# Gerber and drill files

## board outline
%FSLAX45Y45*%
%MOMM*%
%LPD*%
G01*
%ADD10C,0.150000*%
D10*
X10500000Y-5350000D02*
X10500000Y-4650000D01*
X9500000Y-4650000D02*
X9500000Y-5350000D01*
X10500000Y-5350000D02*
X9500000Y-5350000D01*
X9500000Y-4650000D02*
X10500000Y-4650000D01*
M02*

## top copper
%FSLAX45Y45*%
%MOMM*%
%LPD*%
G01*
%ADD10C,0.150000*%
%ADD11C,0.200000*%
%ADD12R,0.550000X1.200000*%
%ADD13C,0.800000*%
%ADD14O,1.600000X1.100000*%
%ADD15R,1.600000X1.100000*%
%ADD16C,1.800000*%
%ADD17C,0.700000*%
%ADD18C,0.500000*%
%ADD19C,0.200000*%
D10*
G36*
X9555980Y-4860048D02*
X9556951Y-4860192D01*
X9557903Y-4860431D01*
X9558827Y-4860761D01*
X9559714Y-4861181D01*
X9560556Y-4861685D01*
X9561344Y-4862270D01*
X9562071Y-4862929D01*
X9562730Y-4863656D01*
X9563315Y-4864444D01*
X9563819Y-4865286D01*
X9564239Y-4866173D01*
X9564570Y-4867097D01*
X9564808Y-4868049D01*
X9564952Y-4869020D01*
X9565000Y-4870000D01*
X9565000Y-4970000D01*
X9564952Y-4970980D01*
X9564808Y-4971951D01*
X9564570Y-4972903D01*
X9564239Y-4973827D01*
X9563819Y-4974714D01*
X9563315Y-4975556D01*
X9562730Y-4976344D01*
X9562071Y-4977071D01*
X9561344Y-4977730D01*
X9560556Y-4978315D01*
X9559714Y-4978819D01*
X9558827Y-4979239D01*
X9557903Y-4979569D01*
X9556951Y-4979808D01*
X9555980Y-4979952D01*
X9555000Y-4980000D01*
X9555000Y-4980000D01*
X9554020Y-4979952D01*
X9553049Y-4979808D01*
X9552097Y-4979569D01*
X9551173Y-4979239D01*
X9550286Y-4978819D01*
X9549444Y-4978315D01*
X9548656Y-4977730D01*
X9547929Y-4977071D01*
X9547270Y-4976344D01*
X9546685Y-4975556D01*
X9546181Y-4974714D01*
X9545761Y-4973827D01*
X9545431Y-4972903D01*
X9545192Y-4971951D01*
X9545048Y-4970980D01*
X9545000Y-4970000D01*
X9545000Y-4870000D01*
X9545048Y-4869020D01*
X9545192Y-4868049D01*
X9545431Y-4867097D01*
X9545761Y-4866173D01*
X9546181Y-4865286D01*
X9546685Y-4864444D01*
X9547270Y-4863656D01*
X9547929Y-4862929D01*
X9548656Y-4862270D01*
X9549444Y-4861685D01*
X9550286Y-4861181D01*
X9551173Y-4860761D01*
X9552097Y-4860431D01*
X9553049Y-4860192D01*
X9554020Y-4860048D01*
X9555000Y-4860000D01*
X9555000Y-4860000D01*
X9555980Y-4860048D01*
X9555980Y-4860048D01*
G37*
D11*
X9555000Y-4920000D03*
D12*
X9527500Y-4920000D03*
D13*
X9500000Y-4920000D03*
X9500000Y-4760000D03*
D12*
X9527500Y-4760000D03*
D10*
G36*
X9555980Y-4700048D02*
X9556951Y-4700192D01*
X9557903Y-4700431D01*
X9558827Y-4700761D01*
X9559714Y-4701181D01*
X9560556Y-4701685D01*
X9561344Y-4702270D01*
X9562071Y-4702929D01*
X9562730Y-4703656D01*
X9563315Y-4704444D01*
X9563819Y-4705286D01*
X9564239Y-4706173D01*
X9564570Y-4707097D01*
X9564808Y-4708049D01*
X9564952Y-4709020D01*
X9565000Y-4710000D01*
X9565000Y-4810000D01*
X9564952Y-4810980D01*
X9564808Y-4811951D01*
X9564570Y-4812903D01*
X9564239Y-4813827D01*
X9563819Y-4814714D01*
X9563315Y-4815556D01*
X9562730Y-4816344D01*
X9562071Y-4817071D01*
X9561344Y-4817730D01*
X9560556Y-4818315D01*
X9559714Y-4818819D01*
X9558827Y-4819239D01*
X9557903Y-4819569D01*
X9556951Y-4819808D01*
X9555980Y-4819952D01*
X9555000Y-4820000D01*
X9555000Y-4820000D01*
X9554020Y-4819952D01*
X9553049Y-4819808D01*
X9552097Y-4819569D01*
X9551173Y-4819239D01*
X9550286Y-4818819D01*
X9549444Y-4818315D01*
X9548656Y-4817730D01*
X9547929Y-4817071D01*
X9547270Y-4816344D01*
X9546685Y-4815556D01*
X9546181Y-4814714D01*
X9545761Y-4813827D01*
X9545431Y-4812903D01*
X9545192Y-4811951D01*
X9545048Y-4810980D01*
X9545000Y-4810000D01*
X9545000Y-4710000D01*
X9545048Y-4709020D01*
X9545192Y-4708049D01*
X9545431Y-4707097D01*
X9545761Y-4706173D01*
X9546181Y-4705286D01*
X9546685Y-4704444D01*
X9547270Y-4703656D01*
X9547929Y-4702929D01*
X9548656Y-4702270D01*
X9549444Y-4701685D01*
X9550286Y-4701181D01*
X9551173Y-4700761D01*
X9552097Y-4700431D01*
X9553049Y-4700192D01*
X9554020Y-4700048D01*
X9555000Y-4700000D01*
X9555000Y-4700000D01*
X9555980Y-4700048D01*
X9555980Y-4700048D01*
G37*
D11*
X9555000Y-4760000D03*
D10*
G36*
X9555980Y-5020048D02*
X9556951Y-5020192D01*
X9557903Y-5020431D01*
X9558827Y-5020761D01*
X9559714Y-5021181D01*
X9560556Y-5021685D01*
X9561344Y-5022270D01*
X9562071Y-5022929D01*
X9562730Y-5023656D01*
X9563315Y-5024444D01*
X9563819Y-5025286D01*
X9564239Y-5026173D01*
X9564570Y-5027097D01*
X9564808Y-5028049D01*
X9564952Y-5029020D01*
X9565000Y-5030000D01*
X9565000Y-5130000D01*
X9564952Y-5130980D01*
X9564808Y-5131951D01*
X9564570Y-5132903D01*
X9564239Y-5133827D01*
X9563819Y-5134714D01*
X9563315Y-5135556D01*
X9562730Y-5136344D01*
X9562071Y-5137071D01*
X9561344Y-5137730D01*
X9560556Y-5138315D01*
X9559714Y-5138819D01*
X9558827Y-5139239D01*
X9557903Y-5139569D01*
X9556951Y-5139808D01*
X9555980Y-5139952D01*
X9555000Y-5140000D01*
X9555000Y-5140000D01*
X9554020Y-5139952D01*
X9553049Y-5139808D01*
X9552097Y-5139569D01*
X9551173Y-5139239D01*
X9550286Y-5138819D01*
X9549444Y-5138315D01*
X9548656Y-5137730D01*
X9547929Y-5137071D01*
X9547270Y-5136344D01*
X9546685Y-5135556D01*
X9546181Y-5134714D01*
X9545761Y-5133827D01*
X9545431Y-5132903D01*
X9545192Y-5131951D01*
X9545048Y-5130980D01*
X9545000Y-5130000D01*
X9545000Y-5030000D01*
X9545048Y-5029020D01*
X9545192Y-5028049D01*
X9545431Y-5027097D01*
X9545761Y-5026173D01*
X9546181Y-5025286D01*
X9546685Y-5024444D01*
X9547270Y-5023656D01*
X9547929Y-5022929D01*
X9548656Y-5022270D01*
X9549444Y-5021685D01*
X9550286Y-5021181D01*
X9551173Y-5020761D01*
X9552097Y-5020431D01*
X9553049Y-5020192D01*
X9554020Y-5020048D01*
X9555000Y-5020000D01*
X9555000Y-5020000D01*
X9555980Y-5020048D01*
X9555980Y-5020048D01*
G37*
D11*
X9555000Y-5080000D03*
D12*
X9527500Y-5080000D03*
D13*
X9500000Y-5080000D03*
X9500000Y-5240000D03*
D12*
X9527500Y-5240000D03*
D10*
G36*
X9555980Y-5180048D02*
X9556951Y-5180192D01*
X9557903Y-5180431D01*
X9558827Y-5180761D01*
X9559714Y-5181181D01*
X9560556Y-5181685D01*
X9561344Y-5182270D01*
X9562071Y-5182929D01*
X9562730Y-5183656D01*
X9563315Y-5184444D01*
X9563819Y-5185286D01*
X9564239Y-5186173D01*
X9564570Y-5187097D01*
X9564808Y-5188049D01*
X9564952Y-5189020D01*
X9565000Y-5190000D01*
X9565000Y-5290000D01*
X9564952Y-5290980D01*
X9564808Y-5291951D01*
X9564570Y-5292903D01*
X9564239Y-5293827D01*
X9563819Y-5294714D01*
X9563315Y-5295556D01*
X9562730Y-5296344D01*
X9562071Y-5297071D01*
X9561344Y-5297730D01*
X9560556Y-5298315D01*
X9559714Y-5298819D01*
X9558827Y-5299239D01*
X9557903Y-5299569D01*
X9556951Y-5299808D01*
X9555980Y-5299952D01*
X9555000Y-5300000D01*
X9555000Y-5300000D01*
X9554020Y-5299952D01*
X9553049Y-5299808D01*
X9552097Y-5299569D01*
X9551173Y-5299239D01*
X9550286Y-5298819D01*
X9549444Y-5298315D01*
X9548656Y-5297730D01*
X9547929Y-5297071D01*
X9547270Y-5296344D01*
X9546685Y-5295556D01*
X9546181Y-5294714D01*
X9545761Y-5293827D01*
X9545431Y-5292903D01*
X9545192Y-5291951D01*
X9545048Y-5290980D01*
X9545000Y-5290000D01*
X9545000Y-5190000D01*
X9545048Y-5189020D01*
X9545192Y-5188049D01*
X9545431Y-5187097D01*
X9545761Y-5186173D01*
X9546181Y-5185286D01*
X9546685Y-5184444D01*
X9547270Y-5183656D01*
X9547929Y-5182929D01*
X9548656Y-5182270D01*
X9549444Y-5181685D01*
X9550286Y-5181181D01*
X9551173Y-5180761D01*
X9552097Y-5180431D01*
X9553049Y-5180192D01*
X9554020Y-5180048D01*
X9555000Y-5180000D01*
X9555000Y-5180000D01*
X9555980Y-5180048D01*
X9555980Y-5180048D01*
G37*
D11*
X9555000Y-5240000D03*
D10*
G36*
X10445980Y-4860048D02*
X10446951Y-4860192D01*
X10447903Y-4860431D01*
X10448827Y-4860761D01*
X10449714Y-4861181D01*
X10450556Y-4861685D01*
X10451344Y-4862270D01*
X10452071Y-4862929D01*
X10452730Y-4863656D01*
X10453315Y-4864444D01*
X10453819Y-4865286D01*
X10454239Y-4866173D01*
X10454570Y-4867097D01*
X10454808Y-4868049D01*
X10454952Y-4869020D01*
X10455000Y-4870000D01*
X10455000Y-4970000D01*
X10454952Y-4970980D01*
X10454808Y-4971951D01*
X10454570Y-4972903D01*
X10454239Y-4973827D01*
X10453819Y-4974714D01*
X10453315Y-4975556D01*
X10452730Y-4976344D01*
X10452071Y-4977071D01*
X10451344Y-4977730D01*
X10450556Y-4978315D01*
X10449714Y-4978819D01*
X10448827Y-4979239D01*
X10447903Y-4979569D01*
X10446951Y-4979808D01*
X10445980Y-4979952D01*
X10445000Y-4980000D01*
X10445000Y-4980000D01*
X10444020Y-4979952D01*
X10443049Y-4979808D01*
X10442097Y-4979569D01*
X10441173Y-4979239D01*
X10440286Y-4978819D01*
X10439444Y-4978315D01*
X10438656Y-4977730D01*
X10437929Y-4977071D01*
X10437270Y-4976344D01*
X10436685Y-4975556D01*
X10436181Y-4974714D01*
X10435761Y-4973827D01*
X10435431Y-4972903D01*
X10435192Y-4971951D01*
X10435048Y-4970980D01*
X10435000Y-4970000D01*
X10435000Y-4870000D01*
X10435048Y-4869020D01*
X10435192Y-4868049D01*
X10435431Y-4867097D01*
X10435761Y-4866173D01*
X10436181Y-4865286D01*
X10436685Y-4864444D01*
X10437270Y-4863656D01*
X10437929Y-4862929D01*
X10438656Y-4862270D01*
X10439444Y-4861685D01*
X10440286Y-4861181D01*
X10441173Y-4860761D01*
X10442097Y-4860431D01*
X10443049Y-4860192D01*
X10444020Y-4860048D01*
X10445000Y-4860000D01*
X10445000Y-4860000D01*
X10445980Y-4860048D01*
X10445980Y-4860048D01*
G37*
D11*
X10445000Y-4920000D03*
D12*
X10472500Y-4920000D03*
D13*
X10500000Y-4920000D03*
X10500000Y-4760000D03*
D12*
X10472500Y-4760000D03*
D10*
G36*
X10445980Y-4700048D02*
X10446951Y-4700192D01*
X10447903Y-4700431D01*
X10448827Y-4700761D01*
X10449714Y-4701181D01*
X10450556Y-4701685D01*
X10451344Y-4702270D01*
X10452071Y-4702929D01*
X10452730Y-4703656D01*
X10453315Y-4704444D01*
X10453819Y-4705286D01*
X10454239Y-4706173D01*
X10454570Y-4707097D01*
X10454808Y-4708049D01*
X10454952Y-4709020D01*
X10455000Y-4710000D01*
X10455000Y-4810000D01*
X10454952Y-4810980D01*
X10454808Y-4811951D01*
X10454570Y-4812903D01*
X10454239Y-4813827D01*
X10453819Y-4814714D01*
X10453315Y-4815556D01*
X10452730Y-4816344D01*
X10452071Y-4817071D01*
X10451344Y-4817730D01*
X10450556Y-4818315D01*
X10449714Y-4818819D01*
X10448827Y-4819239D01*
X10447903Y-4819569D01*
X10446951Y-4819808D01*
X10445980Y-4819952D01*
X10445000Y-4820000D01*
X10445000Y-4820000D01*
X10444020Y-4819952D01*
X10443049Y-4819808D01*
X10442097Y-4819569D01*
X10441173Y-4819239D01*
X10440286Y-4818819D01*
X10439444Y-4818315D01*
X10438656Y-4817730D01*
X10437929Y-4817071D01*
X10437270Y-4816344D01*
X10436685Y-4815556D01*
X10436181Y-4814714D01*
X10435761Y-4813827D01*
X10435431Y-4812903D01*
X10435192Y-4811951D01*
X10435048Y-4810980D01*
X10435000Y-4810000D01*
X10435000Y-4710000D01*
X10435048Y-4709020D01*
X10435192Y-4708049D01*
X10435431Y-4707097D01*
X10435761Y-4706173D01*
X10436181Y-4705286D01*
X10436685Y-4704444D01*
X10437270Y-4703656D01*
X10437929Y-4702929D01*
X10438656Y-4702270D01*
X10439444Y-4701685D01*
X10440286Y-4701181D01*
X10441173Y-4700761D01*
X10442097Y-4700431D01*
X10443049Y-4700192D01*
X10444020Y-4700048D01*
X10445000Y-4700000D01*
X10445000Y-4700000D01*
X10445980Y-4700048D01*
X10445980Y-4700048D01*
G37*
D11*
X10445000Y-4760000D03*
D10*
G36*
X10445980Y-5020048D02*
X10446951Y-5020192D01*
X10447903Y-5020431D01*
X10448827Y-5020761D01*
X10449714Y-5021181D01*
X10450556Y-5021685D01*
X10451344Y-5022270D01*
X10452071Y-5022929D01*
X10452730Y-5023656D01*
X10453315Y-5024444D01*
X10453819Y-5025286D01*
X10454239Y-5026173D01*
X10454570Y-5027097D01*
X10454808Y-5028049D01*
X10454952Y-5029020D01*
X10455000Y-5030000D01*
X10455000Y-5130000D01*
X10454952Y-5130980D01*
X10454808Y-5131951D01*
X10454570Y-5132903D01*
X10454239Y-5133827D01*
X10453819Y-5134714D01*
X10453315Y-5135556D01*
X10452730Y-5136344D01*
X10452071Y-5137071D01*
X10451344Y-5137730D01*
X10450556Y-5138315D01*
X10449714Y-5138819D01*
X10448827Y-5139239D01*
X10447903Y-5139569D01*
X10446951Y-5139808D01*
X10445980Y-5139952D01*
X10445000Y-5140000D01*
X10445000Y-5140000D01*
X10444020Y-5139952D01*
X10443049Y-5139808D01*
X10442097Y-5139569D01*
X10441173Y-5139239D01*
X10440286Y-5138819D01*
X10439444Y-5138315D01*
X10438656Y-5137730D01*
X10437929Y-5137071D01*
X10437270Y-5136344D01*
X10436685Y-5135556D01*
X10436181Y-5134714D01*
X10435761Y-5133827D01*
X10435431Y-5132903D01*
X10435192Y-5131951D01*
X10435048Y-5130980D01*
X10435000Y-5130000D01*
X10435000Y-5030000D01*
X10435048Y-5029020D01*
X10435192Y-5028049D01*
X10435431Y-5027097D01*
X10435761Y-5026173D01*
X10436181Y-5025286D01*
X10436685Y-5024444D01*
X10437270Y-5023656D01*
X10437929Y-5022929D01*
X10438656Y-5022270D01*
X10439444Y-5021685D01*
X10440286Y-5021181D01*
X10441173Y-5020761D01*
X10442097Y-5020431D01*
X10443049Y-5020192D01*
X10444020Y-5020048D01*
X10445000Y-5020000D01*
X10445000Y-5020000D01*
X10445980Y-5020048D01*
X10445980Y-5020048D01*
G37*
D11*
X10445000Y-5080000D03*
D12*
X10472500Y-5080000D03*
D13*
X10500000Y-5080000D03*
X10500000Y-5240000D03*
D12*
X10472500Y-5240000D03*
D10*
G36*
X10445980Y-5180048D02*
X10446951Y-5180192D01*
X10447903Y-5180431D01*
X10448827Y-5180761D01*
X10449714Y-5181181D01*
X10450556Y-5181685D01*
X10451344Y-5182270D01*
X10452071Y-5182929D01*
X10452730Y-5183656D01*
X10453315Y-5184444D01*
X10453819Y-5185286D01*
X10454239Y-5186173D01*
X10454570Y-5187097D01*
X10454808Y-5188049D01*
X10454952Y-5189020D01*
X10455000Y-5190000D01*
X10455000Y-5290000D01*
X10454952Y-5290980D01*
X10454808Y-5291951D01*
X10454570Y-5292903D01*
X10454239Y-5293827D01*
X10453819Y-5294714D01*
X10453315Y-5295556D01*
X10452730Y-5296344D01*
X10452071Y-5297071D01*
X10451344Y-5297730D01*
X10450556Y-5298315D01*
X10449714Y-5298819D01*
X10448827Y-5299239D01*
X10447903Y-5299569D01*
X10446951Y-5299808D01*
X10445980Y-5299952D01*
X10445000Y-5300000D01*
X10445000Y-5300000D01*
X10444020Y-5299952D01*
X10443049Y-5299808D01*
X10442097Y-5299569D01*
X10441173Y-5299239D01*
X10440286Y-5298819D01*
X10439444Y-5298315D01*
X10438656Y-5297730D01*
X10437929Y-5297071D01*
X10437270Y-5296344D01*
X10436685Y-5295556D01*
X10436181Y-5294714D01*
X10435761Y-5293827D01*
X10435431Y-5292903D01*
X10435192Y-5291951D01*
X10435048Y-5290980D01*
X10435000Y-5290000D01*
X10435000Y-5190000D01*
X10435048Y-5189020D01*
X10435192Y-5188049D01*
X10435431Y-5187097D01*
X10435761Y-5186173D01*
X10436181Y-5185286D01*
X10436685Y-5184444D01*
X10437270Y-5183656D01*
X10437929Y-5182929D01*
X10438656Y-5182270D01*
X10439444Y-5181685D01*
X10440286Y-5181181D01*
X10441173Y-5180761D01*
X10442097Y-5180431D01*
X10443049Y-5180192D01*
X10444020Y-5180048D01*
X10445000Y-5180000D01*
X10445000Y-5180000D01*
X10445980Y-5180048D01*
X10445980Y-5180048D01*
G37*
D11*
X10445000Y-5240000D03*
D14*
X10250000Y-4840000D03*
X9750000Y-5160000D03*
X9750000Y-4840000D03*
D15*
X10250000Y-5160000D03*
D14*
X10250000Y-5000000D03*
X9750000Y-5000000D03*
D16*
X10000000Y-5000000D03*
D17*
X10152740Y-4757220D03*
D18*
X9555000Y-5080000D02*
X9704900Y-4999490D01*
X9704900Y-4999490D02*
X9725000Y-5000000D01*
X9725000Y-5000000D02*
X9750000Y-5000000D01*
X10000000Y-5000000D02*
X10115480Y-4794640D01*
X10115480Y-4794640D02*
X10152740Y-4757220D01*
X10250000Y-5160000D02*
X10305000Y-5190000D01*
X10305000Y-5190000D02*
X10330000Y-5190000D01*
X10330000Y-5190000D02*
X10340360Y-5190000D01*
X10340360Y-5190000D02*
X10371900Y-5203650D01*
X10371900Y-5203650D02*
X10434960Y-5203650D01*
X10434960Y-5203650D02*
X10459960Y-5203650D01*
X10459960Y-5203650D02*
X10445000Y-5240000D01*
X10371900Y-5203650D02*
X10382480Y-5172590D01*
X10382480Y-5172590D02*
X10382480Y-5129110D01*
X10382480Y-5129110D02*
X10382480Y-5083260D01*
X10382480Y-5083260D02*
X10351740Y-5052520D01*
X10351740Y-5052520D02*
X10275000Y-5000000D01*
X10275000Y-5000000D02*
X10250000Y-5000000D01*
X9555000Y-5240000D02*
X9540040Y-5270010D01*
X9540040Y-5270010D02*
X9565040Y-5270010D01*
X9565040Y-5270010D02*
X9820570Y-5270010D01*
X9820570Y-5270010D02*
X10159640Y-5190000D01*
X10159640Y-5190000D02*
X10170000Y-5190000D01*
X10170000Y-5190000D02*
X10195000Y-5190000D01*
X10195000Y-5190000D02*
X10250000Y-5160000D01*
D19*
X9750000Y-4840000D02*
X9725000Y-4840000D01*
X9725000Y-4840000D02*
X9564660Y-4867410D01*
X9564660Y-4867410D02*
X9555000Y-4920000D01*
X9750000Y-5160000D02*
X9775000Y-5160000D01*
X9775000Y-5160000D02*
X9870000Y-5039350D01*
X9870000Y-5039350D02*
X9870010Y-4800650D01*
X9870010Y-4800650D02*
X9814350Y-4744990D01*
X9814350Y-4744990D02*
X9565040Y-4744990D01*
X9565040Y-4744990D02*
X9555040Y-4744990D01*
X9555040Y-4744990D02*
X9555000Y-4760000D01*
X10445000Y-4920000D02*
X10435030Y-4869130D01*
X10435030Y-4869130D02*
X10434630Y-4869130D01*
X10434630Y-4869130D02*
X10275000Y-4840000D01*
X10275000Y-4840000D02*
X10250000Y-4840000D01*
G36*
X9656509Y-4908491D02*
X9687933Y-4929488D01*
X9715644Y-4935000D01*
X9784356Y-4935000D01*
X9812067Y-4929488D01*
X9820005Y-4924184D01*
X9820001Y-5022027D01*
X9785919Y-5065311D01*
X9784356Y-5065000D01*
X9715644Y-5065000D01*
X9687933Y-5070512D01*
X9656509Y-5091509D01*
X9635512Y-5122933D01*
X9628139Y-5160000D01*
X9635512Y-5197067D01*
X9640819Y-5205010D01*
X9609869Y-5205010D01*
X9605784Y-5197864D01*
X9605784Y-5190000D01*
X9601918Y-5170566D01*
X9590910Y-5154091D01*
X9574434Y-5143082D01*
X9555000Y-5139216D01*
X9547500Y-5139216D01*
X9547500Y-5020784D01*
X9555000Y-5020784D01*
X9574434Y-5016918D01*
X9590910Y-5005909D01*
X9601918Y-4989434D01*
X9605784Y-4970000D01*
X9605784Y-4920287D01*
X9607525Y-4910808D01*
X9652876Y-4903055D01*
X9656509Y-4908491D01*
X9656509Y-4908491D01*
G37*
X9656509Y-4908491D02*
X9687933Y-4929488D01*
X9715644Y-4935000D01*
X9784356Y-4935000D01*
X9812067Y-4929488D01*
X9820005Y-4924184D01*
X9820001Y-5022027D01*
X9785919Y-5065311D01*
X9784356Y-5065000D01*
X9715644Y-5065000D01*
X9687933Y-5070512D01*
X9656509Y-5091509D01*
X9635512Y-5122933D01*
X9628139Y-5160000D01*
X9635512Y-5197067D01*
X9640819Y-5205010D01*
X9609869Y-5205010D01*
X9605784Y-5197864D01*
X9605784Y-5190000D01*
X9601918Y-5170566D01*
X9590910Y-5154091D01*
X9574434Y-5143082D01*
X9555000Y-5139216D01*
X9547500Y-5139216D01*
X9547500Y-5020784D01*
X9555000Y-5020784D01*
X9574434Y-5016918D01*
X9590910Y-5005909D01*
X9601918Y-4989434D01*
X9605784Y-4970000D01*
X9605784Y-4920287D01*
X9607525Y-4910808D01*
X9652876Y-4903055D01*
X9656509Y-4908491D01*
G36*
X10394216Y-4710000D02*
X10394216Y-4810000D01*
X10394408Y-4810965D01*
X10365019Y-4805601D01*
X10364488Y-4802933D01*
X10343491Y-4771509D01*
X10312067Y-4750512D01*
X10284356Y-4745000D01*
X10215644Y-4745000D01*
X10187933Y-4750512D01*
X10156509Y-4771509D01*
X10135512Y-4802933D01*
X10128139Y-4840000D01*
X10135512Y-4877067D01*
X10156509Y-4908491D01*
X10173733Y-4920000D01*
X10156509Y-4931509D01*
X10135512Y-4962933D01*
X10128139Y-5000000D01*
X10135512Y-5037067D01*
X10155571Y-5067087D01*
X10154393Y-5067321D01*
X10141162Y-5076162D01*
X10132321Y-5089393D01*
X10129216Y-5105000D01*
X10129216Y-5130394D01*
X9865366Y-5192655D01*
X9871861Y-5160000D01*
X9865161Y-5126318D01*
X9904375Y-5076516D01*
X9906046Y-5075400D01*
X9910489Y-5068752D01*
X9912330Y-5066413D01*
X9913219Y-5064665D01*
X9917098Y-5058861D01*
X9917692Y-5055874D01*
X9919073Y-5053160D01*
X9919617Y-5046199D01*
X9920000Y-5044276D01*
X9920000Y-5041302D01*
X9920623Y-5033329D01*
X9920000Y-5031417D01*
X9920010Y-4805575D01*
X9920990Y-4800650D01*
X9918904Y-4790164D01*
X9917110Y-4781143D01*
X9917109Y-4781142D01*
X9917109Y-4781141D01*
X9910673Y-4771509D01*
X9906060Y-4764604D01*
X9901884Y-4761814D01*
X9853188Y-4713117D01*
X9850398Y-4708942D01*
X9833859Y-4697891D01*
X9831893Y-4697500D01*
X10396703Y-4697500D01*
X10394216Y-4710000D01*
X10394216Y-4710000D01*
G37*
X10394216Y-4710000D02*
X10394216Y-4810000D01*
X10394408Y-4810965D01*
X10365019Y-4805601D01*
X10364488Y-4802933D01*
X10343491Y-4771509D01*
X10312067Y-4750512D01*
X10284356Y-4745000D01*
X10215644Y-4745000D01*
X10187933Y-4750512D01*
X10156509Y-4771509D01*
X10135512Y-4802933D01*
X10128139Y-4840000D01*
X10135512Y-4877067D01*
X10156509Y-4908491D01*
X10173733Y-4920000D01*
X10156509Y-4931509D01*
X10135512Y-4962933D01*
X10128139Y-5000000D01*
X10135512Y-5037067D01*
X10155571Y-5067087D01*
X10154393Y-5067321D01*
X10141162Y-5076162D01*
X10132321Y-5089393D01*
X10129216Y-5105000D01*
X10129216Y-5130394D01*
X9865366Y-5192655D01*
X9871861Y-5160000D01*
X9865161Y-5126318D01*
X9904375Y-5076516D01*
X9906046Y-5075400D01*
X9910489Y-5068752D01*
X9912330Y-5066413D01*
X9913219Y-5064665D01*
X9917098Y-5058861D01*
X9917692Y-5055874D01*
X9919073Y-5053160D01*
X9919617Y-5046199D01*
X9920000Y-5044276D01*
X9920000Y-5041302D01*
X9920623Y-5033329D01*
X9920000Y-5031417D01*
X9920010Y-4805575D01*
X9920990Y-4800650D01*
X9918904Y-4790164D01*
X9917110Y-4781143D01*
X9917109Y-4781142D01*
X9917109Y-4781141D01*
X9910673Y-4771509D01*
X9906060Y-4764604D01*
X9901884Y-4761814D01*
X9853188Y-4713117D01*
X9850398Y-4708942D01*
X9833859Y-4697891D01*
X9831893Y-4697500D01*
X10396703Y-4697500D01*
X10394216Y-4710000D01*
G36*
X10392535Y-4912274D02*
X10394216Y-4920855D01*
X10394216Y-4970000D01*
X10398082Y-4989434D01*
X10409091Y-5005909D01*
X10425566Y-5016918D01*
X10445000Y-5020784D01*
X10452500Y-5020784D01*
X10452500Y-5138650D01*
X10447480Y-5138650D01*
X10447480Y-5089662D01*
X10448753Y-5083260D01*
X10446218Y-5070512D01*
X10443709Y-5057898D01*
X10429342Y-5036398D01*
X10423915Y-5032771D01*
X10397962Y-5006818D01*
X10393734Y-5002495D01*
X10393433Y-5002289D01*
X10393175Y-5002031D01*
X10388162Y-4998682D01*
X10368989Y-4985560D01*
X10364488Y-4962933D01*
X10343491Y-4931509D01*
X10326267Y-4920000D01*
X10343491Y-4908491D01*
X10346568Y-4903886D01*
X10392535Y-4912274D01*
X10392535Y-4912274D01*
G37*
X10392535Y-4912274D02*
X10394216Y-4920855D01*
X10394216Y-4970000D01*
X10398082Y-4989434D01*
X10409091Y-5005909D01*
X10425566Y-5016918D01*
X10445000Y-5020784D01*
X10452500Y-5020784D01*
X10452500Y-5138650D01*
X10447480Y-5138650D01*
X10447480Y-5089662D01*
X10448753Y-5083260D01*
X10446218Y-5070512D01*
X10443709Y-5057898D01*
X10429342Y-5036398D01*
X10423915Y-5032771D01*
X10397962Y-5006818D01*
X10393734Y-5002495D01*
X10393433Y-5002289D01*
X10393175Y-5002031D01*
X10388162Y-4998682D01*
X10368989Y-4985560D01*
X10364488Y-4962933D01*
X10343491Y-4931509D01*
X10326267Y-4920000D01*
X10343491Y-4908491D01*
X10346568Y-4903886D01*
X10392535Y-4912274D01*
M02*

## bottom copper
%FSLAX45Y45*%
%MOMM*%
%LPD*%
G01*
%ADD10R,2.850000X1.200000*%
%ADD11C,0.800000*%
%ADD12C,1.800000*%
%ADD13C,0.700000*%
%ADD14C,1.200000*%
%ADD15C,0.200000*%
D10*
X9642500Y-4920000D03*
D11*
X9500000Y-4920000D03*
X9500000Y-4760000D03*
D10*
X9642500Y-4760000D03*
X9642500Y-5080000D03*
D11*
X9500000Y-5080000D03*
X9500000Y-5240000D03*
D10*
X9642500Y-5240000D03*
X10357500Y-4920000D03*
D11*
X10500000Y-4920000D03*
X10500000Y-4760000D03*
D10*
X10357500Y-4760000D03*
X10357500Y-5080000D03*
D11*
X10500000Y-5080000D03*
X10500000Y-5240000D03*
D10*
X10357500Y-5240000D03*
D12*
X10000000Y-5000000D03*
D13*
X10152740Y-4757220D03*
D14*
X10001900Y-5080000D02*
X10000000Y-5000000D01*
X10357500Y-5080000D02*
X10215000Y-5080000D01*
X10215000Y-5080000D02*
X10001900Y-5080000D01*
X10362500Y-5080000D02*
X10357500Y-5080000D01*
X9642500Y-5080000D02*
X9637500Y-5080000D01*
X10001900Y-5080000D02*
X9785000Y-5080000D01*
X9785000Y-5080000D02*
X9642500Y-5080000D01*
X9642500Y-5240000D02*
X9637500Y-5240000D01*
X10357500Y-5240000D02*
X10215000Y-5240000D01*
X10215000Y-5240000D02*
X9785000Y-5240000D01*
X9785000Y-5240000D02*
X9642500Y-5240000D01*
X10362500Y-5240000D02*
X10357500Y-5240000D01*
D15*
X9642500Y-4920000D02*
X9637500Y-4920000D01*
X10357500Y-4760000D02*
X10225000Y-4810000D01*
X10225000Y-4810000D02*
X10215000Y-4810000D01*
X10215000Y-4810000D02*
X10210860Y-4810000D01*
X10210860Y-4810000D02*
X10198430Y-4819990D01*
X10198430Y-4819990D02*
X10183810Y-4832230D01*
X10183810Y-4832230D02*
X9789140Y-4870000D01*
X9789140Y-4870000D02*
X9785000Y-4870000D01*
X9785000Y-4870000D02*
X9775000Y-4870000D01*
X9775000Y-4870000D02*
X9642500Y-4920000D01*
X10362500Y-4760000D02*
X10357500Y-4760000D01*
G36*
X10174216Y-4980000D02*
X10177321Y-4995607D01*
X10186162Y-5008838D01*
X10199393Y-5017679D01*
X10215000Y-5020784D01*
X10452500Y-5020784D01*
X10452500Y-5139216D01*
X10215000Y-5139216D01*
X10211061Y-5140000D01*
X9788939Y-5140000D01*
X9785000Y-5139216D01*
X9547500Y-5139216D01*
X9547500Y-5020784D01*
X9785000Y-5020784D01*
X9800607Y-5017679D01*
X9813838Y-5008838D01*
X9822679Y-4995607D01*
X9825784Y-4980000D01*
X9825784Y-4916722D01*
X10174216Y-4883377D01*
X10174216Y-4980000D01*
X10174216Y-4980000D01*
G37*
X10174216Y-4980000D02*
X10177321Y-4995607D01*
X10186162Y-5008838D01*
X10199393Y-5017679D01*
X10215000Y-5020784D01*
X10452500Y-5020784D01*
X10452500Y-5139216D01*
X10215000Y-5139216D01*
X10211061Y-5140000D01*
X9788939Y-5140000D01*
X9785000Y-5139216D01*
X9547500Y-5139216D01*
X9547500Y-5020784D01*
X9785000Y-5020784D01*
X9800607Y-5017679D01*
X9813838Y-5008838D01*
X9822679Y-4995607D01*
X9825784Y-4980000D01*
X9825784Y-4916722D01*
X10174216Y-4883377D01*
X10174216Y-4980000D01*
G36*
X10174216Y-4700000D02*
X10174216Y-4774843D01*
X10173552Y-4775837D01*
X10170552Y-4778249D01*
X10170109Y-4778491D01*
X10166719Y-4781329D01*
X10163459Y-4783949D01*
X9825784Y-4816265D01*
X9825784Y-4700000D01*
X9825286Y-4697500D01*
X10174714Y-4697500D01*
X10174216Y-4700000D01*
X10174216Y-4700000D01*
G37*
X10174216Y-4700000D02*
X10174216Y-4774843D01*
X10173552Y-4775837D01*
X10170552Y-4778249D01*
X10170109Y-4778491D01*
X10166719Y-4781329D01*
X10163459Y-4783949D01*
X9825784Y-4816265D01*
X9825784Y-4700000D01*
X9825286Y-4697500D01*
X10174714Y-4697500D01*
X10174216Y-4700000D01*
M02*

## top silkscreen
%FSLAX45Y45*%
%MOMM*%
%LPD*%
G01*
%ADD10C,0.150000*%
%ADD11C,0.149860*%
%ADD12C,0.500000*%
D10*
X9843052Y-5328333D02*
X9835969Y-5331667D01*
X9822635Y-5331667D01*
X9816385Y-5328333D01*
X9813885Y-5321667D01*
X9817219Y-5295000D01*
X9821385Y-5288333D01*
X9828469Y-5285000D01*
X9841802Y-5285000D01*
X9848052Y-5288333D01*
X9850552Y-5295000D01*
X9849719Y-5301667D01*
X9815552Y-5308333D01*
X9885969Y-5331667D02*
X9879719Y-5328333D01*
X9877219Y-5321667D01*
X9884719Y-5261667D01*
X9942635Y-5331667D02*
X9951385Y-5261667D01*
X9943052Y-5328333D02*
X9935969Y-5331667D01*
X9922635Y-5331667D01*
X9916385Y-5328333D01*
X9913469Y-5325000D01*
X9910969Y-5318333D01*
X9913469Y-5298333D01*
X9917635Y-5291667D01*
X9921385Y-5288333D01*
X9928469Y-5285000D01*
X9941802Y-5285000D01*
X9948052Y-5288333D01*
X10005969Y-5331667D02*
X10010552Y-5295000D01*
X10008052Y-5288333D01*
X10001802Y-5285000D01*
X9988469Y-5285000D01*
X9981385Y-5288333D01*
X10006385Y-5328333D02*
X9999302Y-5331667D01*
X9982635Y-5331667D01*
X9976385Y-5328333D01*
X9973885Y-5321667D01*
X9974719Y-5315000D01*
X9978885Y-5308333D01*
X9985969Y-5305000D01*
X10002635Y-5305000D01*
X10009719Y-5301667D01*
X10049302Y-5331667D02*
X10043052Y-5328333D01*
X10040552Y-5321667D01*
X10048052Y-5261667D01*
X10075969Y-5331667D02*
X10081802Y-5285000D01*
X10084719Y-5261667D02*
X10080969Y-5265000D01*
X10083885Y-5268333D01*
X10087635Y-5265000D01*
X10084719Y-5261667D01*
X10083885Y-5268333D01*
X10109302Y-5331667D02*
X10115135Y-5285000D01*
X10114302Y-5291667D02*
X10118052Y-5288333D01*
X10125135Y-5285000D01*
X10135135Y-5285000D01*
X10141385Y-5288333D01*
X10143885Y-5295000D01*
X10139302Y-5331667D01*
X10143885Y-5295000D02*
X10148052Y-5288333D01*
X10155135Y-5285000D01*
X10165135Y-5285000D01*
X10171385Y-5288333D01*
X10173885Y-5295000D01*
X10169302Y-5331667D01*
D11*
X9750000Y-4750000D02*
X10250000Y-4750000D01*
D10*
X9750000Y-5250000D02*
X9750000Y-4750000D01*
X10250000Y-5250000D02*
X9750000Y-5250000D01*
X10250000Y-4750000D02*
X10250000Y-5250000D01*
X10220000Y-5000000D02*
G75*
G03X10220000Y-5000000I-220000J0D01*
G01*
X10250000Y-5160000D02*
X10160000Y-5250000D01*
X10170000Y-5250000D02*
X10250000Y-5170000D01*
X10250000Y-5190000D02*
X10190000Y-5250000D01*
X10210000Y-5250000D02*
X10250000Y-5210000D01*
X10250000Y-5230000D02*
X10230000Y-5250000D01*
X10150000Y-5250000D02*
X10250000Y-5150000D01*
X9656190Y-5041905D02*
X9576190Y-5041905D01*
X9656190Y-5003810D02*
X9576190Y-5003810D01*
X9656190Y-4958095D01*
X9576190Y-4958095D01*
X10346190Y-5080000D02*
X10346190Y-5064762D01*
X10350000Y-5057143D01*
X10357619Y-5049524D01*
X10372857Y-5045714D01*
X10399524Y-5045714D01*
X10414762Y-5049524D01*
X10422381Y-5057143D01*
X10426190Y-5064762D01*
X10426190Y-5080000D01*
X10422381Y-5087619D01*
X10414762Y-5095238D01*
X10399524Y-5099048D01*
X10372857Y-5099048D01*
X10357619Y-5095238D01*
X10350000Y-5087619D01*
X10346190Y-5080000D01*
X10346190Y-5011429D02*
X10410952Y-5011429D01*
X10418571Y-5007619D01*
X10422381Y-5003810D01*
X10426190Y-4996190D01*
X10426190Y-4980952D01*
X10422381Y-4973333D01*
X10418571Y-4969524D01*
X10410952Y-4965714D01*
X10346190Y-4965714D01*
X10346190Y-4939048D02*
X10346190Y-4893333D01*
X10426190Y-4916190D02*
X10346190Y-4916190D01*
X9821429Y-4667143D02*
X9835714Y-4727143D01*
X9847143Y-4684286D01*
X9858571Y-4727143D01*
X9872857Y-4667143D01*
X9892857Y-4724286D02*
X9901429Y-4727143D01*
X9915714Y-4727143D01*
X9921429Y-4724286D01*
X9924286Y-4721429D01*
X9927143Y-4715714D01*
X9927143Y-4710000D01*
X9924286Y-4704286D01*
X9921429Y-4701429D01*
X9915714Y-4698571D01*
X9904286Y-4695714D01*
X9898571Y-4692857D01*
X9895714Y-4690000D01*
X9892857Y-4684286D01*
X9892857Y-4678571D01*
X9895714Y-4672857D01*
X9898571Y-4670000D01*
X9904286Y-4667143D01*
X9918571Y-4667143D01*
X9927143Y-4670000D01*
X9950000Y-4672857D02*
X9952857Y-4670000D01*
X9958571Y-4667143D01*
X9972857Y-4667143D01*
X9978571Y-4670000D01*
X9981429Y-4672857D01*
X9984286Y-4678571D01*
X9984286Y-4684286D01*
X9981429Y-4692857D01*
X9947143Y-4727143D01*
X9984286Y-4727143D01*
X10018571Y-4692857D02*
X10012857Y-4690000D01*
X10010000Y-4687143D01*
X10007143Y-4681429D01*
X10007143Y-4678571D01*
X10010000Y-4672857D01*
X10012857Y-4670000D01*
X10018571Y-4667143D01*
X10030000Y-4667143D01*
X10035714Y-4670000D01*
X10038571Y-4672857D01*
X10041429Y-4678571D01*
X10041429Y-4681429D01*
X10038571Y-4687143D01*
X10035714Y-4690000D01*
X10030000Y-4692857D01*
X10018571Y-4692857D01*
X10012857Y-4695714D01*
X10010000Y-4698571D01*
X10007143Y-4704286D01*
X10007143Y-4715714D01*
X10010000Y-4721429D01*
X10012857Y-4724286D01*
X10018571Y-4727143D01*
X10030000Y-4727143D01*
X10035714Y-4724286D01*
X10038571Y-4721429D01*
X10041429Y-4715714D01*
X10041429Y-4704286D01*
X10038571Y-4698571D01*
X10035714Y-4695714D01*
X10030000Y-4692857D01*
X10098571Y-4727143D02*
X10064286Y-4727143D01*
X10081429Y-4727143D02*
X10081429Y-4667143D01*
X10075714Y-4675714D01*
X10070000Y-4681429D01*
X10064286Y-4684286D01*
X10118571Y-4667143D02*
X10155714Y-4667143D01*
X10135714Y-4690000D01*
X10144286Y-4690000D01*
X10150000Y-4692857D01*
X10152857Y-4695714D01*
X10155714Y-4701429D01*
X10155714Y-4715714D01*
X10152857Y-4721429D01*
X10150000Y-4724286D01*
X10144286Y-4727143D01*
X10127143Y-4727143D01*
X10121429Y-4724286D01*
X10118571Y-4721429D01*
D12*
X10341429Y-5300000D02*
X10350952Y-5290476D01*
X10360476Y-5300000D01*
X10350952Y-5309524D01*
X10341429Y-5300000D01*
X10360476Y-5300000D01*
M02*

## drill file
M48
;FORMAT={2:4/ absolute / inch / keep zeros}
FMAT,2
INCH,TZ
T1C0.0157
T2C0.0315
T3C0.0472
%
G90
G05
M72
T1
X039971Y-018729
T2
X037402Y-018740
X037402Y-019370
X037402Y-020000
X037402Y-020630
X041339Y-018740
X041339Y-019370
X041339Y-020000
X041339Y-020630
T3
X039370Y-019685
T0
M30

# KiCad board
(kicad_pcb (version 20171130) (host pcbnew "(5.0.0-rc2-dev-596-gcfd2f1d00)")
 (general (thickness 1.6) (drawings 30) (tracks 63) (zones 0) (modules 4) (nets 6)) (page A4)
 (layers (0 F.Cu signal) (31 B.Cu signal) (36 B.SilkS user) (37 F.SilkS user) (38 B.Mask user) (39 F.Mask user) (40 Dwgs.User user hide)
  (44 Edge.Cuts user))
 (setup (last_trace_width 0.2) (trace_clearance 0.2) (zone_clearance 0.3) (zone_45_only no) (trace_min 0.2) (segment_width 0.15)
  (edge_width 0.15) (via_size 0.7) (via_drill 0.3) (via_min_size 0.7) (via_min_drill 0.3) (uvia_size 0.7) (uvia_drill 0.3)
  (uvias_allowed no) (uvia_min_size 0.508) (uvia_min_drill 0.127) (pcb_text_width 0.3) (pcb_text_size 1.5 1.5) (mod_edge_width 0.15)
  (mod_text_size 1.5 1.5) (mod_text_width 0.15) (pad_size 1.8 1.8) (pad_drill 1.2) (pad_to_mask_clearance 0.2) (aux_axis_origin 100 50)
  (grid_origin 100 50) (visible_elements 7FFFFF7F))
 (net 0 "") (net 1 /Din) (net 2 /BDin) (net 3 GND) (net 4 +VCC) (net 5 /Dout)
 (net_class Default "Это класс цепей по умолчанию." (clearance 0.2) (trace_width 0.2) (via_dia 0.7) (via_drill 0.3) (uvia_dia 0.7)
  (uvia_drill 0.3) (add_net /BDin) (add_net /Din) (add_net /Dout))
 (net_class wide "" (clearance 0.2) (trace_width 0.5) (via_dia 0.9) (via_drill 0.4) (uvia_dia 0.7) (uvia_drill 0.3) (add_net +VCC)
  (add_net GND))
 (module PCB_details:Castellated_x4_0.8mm (layer F.Cu) (at 95 52.4 90)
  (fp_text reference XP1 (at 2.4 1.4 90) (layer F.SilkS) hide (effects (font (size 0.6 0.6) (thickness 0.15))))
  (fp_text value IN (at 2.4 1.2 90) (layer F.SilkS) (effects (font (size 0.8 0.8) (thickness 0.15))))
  (pad 3 smd roundrect (at 3.2 0.55 90) (size 1.2 0.2) (layers F.Cu F.Mask) (roundrect_rratio 0.5) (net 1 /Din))
  (pad 3 smd rect (at 3.2 1.425 90) (size 1.2 2.85) (layers B.Cu B.Mask) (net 1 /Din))
  (pad 3 smd rect (at 3.2 0.275 90) (size 1.2 0.55) (layers F.Cu F.Mask) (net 1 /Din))
  (pad 3 thru_hole circle (at 3.2 0 90) (size 0.8 0.8) (drill 0.8) (layers *.Cu) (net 1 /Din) (clearance 0.001))
  (pad 4 thru_hole circle (at 4.8 0 90) (size 0.8 0.8) (drill 0.8) (layers *.Cu) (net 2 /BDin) (clearance 0.001))
  (pad 4 smd rect (at 4.8 0.275 90) (size 1.2 0.55) (layers F.Cu F.Mask) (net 2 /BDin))
  (pad 4 smd rect (at 4.8 1.425 90) (size 1.2 2.85) (layers B.Cu B.Mask) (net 2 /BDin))
  (pad 4 smd roundrect (at 4.8 0.55 90) (size 1.2 0.2) (layers F.Cu F.Mask) (roundrect_rratio 0.5) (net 2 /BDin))
  (pad 2 smd roundrect (at 1.6 0.55 90) (size 1.2 0.2) (layers F.Cu F.Mask) (roundrect_rratio 0.5) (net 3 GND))
  (pad 2 smd rect (at 1.6 1.425 90) (size 1.2 2.85) (layers B.Cu B.Mask) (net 3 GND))
  (pad 2 smd rect (at 1.6 0.275 90) (size 1.2 0.55) (layers F.Cu F.Mask) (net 3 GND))
  (pad 2 thru_hole circle (at 1.6 0 90) (size 0.8 0.8) (drill 0.8) (layers *.Cu) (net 3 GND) (clearance 0.001))
  (pad 1 thru_hole circle (at 0 0 90) (size 0.8 0.8) (drill 0.8) (layers *.Cu) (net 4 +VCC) (clearance 0.001))
  (pad 1 smd rect (at 0 0.275 90) (size 1.2 0.55) (layers F.Cu F.Mask) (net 4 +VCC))
  (pad 1 smd rect (at 0 1.425 90) (size 1.2 2.85) (layers B.Cu B.Mask) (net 4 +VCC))
  (pad 1 smd roundrect (at 0 0.55 90) (size 1.2 0.2) (layers F.Cu F.Mask) (roundrect_rratio 0.5) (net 4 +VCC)))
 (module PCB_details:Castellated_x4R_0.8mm (layer F.Cu) (at 105 52.4 270)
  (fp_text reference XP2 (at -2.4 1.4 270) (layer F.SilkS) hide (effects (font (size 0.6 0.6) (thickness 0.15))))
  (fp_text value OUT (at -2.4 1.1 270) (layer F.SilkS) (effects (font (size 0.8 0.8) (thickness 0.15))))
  (pad 3 smd roundrect (at -3.2 0.55 270) (size 1.2 0.2) (layers F.Cu F.Mask) (roundrect_rratio 0.5) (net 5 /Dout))
  (pad 3 smd rect (at -3.2 1.425 270) (size 1.2 2.85) (layers B.Cu B.Mask) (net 5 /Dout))
  (pad 3 smd rect (at -3.2 0.275 270) (size 1.2 0.55) (layers F.Cu F.Mask) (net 5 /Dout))
  (pad 3 thru_hole circle (at -3.2 0 270) (size 0.8 0.8) (drill 0.8) (layers *.Cu) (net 5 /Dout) (clearance 0.001))
  (pad 4 thru_hole circle (at -4.8 0 270) (size 0.8 0.8) (drill 0.8) (layers *.Cu) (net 1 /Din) (clearance 0.001))
  (pad 4 smd rect (at -4.8 0.275 270) (size 1.2 0.55) (layers F.Cu F.Mask) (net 1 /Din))
  (pad 4 smd rect (at -4.8 1.425 270) (size 1.2 2.85) (layers B.Cu B.Mask) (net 1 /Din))
  (pad 4 smd roundrect (at -4.8 0.55 270) (size 1.2 0.2) (layers F.Cu F.Mask) (roundrect_rratio 0.5) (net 1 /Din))
  (pad 2 smd roundrect (at -1.6 0.55 270) (size 1.2 0.2) (layers F.Cu F.Mask) (roundrect_rratio 0.5) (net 3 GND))
  (pad 2 smd rect (at -1.6 1.425 270) (size 1.2 2.85) (layers B.Cu B.Mask) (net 3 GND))
  (pad 2 smd rect (at -1.6 0.275 270) (size 1.2 0.55) (layers F.Cu F.Mask) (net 3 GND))
  (pad 2 thru_hole circle (at -1.6 0 270) (size 0.8 0.8) (drill 0.8) (layers *.Cu) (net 3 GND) (clearance 0.001))
  (pad 1 thru_hole circle (at 0 0 270) (size 0.8 0.8) (drill 0.8) (layers *.Cu) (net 4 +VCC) (clearance 0.001))
  (pad 1 smd rect (at 0 0.275 270) (size 1.2 0.55) (layers F.Cu F.Mask) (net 4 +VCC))
  (pad 1 smd rect (at 0 1.425 270) (size 1.2 2.85) (layers B.Cu B.Mask) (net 4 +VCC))
  (pad 1 smd roundrect (at 0 0.55 270) (size 1.2 0.2) (layers F.Cu F.Mask) (roundrect_rratio 0.5) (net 4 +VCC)))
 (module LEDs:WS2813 (layer F.Cu) (at 100 50)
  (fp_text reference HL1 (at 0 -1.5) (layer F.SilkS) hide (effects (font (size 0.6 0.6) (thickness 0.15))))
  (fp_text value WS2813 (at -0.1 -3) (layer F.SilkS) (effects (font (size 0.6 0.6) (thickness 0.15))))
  (fp_line (start -2.5 -2.5) (end 2.5 -2.5) (layer F.SilkS) (width 0.14986))
  (fp_line (start -2.5 2.5) (end -2.5 -2.5) (layer F.SilkS) (width 0.15))
  (fp_line (start 2.5 2.5) (end -2.5 2.5) (layer F.SilkS) (width 0.15))
  (fp_line (start 2.5 -2.5) (end 2.5 2.5) (layer F.SilkS) (width 0.15))
  (fp_circle (center 0 0) (end 0 2.2) (layer F.SilkS) (width 0.15))
  (fp_line (start 2.5 1.6) (end 1.6 2.5) (layer F.SilkS) (width 0.15))
  (fp_line (start 1.7 2.5) (end 2.5 1.7) (layer F.SilkS) (width 0.15))
  (fp_line (start 2.5 1.9) (end 1.9 2.5) (layer F.SilkS) (width 0.15))
  (fp_line (start 2.1 2.5) (end 2.5 2.1) (layer F.SilkS) (width 0.15))
  (fp_line (start 2.5 2.3) (end 2.3 2.5) (layer F.SilkS) (width 0.15))
  (fp_line (start 1.5 2.5) (end 2.5 1.5) (layer F.SilkS) (width 0.15))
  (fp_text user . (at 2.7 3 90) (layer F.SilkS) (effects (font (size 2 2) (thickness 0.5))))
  (pad 3 smd oval (at 2.5 -1.6) (size 1.6 1.1) (layers F.Cu F.Mask) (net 5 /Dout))
  (pad 6 smd oval (at -2.5 1.6) (size 1.6 1.1) (layers F.Cu F.Mask) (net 2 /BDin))
  (pad 4 smd oval (at -2.5 -1.6) (size 1.6 1.1) (layers F.Cu F.Mask) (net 1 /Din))
  (pad 1 smd rect (at 2.5 1.6) (size 1.6 1.1) (layers F.Cu F.Mask) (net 4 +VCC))
  (pad 2 smd oval (at 2.5 0) (size 1.6 1.1) (layers F.Cu F.Mask) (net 4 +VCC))
  (pad 5 smd oval (at -2.5 0) (size 1.6 1.1) (layers F.Cu F.Mask) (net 3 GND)))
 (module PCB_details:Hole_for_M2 (layer F.Cu) (at 100 50 270)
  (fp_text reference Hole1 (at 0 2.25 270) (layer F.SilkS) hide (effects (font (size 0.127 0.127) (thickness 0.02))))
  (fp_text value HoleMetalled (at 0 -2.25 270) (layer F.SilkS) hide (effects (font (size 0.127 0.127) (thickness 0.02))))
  (pad H thru_hole circle (at 0 0 270) (size 1.8 1.8) (drill 1.2) (layers *.Cu *.Mask) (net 3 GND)))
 (gr_line (start 105 53.5) (end 105 46.5) (angle 90) (layer Edge.Cuts) (width 0.15))
 (gr_line (start 95 46.5) (end 95 53.5) (angle 90) (layer Edge.Cuts) (width 0.15))
 (gr_line (start 105 53.5) (end 95 53.5) (angle 90) (layer Edge.Cuts) (width 0.15))
 (gr_line (start 95 46.5) (end 105 46.5) (angle 90) (layer Edge.Cuts) (width 0.15))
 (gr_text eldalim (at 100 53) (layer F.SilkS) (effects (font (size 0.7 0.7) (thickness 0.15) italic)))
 (segment (start 95.55 50.8) (end 97.049 49.9949) (width 0.5) (layer F.Cu) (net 3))
 (segment (start 97.049 49.9949) (end 97.25 50) (width 0.5) (layer F.Cu) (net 3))
 (segment (start 97.25 50) (end 97.5 50) (width 0.5) (layer F.Cu) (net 3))
 (segment (start 100 50) (end 101.1548 47.9464) (width 0.5) (layer F.Cu) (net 3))
 (segment (start 101.1548 47.9464) (end 101.5274 47.5722) (width 0.5) (layer F.Cu) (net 3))
 (segment (start 100.019 50.8) (end 100 50) (width 1.2) (layer B.Cu) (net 3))
 (segment (start 103.575 50.8) (end 102.15 50.8) (width 1.2) (layer B.Cu) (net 3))
 (segment (start 102.15 50.8) (end 100.019 50.8) (width 1.2) (layer B.Cu) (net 3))
 (segment (start 103.625 50.8) (end 103.575 50.8) (width 1.2) (layer B.Cu) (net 3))
 (segment (start 96.425 50.8) (end 96.375 50.8) (width 1.2) (layer B.Cu) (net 3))
 (segment (start 100.019 50.8) (end 97.85 50.8) (width 1.2) (layer B.Cu) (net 3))
 (segment (start 97.85 50.8) (end 96.425 50.8) (width 1.2) (layer B.Cu) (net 3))
 (via (at 101.5274 47.5722) (size 0.7) (layers F.Cu B.Cu) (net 3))
 (segment (start 102.5 51.6) (end 103.05 51.9) (width 0.5) (layer F.Cu) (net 4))
 (segment (start 103.05 51.9) (end 103.3 51.9) (width 0.5) (layer F.Cu) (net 4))
 (segment (start 103.3 51.9) (end 103.4036 51.9) (width 0.5) (layer F.Cu) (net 4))
 (segment (start 103.4036 51.9) (end 103.719 52.0365) (width 0.5) (layer F.Cu) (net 4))
 (segment (start 103.719 52.0365) (end 104.3496 52.0365) (width 0.5) (layer F.Cu) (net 4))
 (segment (start 104.3496 52.0365) (end 104.5996 52.0365) (width 0.5) (layer F.Cu) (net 4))
 (segment (start 104.5996 52.0365) (end 104.45 52.4) (width 0.5) (layer F.Cu) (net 4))
 (segment (start 103.719 52.0365) (end 103.8248 51.7259) (width 0.5) (layer F.Cu) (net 4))
 (segment (start 103.8248 51.7259) (end 103.8248 51.2911) (width 0.5) (layer F.Cu) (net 4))
 (segment (start 103.8248 51.2911) (end 103.8248 50.8326) (width 0.5) (layer F.Cu) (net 4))
 (segment (start 103.8248 50.8326) (end 103.5174 50.5252) (width 0.5) (layer F.Cu) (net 4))
 (segment (start 103.5174 50.5252) (end 102.75 50) (width 0.5) (layer F.Cu) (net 4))
 (segment (start 102.75 50) (end 102.5 50) (width 0.5) (layer F.Cu) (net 4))
 (segment (start 95.55 52.4) (end 95.4004 52.7001) (width 0.5) (layer F.Cu) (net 4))
 (segment (start 95.4004 52.7001) (end 95.6504 52.7001) (width 0.5) (layer F.Cu) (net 4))
 (segment (start 95.6504 52.7001) (end 98.2057 52.7001) (width 0.5) (layer F.Cu) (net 4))
 (segment (start 98.2057 52.7001) (end 101.5964 51.9) (width 0.5) (layer F.Cu) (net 4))
 (segment (start 101.5964 51.9) (end 101.7 51.9) (width 0.5) (layer F.Cu) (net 4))
 (segment (start 101.7 51.9) (end 101.95 51.9) (width 0.5) (layer F.Cu) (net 4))
 (segment (start 101.95 51.9) (end 102.5 51.6) (width 0.5) (layer F.Cu) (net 4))
 (segment (start 96.425 52.4) (end 96.375 52.4) (width 1.2) (layer B.Cu) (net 4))
 (segment (start 103.575 52.4) (end 102.15 52.4) (width 1.2) (layer B.Cu) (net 4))
 (segment (start 102.15 52.4) (end 97.85 52.4) (width 1.2) (layer B.Cu) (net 4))
 (segment (start 97.85 52.4) (end 96.425 52.4) (width 1.2) (layer B.Cu) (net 4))
 (segment (start 103.625 52.4) (end 103.575 52.4) (width 1.2) (layer B.Cu) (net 4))
 (segment (start 97.5 48.4) (end 97.25 48.4) (width 0.2) (layer F.Cu) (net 1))
 (segment (start 97.25 48.4) (end 95.6466 48.6741) (width 0.2) (layer F.Cu) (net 1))
 (segment (start 95.6466 48.6741) (end 95.55 49.2) (width 0.2) (layer F.Cu) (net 1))
 (segment (start 96.425 49.2) (end 96.375 49.2) (width 0.2) (layer B.Cu) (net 1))
 (segment (start 103.575 47.6) (end 102.25 48.1) (width 0.2) (layer B.Cu) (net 1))
 (segment (start 102.25 48.1) (end 102.15 48.1) (width 0.2) (layer B.Cu) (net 1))
 (segment (start 102.15 48.1) (end 102.1086 48.1) (width 0.2) (layer B.Cu) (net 1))
 (segment (start 102.1086 48.1) (end 101.9843 48.1999) (width 0.2) (layer B.Cu) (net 1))
 (segment (start 101.9843 48.1999) (end 101.8381 48.3223) (width 0.2) (layer B.Cu) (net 1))
 (segment (start 101.8381 48.3223) (end 97.8914 48.7) (width 0.2) (layer B.Cu) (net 1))
 (segment (start 97.8914 48.7) (end 97.85 48.7) (width 0.2) (layer B.Cu) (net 1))
 (segment (start 97.85 48.7) (end 97.75 48.7) (width 0.2) (layer B.Cu) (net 1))
 (segment (start 97.75 48.7) (end 96.425 49.2) (width 0.2) (layer B.Cu) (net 1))
 (segment (start 103.625 47.6) (end 103.575 47.6) (width 0.2) (layer B.Cu) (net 1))
 (segment (start 97.5 51.6) (end 97.75 51.6) (width 0.2) (layer F.Cu) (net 2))
 (segment (start 97.75 51.6) (end 98.7 50.3935) (width 0.2) (layer F.Cu) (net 2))
 (segment (start 98.7 50.3935) (end 98.7001 48.0065) (width 0.2) (layer F.Cu) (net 2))
 (segment (start 98.7001 48.0065) (end 98.1435 47.4499) (width 0.2) (layer F.Cu) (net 2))
 (segment (start 98.1435 47.4499) (end 95.6504 47.4499) (width 0.2) (layer F.Cu) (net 2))
 (segment (start 95.6504 47.4499) (end 95.5504 47.4499) (width 0.2) (layer F.Cu) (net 2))
 (segment (start 95.5504 47.4499) (end 95.55 47.6) (width 0.2) (layer F.Cu) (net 2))
 (segment (start 104.45 49.2) (end 104.3503 48.6913) (width 0.2) (layer F.Cu) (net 5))
 (segment (start 104.3503 48.6913) (end 104.3463 48.6913) (width 0.2) (layer F.Cu) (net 5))
 (segment (start 104.3463 48.6913) (end 102.75 48.4) (width 0.2) (layer F.Cu) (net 5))
 (segment (start 102.75 48.4) (end 102.5 48.4) (width 0.2) (layer F.Cu) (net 5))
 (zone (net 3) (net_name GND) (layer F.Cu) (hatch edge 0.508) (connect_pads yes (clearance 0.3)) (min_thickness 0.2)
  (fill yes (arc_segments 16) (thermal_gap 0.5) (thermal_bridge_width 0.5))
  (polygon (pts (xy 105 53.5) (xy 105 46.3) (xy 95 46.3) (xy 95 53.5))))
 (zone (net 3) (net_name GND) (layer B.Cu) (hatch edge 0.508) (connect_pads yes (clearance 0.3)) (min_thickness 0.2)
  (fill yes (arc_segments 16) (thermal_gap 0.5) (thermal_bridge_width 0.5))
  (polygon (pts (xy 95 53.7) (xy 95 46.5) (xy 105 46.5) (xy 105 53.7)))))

